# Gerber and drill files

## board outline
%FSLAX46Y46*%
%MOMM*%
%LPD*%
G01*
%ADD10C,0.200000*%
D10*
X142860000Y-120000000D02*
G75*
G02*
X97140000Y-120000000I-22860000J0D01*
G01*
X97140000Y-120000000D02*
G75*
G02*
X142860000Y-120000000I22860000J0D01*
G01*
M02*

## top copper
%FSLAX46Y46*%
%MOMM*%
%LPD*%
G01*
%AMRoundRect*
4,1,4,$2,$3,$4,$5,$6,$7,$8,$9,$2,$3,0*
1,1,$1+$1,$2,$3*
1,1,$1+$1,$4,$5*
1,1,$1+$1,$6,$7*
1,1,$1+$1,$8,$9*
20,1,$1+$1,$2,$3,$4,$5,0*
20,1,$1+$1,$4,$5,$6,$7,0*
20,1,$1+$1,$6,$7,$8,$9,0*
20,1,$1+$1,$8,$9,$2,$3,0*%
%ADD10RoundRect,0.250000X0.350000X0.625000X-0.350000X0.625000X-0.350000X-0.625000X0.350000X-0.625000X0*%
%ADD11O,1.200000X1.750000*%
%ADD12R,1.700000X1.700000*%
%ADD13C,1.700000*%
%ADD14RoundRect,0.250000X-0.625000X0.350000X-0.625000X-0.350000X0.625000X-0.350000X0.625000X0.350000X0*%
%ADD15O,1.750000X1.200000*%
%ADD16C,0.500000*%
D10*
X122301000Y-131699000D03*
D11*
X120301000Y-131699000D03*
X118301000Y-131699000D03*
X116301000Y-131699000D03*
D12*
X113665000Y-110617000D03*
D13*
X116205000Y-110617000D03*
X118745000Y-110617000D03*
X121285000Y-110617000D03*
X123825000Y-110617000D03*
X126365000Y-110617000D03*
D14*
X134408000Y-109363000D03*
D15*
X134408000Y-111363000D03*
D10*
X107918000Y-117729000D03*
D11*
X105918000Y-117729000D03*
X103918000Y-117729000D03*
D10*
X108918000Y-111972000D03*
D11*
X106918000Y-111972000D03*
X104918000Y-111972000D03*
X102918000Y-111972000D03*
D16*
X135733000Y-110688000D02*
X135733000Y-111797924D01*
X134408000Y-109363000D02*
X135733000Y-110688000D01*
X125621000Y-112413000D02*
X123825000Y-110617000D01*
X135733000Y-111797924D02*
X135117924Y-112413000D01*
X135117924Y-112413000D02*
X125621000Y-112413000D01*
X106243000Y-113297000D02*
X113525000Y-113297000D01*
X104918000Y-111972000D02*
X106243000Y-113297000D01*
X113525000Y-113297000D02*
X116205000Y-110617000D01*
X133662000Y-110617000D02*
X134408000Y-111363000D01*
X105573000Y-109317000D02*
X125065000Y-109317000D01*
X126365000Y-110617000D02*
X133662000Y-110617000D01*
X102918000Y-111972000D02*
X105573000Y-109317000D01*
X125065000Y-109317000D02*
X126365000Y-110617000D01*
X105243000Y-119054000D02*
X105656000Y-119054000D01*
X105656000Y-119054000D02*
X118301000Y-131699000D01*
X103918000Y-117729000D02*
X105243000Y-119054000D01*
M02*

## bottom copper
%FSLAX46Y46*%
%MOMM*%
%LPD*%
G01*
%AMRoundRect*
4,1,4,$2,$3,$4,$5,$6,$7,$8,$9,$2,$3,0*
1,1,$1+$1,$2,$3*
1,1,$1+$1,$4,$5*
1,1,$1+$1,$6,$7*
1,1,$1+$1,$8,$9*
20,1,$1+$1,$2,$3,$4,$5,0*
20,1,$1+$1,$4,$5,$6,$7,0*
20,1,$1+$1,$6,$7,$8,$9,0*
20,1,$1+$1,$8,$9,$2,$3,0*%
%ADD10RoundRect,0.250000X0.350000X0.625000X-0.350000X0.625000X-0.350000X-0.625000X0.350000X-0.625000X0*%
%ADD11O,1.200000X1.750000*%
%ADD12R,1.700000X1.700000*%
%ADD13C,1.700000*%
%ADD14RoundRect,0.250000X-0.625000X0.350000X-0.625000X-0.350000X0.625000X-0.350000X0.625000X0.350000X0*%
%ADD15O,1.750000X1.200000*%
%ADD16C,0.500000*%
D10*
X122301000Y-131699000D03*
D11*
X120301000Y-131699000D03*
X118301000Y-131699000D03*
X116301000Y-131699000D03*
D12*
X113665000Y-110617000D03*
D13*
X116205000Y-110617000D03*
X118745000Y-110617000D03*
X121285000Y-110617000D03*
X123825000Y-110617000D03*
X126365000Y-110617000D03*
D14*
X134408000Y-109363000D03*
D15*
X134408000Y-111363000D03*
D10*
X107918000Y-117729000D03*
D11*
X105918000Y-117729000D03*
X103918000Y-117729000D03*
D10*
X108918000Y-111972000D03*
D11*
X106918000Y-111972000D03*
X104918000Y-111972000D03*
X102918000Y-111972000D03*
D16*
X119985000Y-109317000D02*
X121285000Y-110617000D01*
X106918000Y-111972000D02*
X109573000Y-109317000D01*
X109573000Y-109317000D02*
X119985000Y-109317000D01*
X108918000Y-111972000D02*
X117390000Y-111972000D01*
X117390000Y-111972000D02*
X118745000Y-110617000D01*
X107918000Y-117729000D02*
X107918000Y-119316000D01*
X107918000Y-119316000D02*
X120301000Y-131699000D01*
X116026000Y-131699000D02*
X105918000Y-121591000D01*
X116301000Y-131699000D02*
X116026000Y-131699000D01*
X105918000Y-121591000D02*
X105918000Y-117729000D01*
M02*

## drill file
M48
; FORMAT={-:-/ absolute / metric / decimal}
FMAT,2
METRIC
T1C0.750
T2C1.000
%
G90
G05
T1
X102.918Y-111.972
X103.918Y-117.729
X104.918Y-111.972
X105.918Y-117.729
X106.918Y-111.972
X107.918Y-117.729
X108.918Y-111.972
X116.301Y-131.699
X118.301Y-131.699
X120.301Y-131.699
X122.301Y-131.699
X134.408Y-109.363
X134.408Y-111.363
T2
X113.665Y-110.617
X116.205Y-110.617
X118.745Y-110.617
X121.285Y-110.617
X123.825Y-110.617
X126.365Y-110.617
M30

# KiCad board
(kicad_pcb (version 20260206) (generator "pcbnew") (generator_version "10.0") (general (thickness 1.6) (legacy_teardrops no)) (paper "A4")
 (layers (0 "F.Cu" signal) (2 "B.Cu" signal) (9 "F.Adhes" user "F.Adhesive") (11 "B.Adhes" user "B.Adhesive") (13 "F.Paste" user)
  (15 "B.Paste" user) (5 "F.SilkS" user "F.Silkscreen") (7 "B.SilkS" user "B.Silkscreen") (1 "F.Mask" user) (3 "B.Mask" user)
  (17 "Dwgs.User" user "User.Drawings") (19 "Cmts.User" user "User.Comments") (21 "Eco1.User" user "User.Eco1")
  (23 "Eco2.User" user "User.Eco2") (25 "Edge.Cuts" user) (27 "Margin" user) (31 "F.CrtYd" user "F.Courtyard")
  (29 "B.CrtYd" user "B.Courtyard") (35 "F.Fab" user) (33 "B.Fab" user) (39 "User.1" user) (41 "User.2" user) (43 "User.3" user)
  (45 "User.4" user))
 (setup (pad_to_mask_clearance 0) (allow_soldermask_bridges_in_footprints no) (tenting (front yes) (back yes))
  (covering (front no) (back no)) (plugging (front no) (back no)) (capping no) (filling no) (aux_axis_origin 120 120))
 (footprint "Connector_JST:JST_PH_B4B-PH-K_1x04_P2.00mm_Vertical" (layer "F.Cu") (at 122.301 131.699 180)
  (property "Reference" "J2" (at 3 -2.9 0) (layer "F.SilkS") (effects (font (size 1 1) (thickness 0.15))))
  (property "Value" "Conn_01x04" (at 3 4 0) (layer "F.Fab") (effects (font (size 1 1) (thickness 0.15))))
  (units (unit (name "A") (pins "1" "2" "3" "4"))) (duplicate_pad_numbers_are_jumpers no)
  (pad "1" thru_hole roundrect (at 0 0 180) (size 1.2 1.75) (drill 0.75) (layers "*.Cu" "*.Mask") (remove_unused_layers no)
   (roundrect_rratio 0.208333) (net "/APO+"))
  (pad "2" thru_hole oval (at 2 0 180) (size 1.2 1.75) (drill 0.75) (layers "*.Cu" "*.Mask") (remove_unused_layers no) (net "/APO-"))
  (pad "3" thru_hole oval (at 4 0 180) (size 1.2 1.75) (drill 0.75) (layers "*.Cu" "*.Mask") (remove_unused_layers no) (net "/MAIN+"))
  (pad "4" thru_hole oval (at 6 0 180) (size 1.2 1.75) (drill 0.75) (layers "*.Cu" "*.Mask") (remove_unused_layers no) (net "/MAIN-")))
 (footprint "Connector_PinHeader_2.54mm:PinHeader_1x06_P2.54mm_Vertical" (layer "F.Cu") (at 113.665 110.617 90)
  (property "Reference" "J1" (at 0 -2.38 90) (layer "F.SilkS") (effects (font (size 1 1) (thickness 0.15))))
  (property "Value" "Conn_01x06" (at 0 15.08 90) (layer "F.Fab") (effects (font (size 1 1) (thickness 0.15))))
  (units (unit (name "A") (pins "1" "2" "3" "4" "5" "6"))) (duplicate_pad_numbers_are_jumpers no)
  (pad "1" thru_hole rect (at 0 0 90) (size 1.7 1.7) (drill 1) (layers "*.Cu" "*.Mask") (remove_unused_layers no) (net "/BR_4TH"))
  (pad "2" thru_hole circle (at 0 2.54 90) (size 1.7 1.7) (drill 1) (layers "*.Cu" "*.Mask") (remove_unused_layers no) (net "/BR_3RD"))
  (pad "3" thru_hole circle (at 0 5.08 90) (size 1.7 1.7) (drill 1) (layers "*.Cu" "*.Mask") (remove_unused_layers no) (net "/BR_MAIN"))
  (pad "4" thru_hole circle (at 0 7.62 90) (size 1.7 1.7) (drill 1) (layers "*.Cu" "*.Mask") (remove_unused_layers no) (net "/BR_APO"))
  (pad "5" thru_hole circle (at 0 10.16 90) (size 1.7 1.7) (drill 1) (layers "*.Cu" "*.Mask") (remove_unused_layers no) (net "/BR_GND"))
  (pad "6" thru_hole circle (at 0 12.7 90) (size 1.7 1.7) (drill 1) (layers "*.Cu" "*.Mask") (remove_unused_layers no) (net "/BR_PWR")))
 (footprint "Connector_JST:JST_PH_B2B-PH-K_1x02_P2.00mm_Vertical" (layer "F.Cu") (at 134.408 109.363 -90)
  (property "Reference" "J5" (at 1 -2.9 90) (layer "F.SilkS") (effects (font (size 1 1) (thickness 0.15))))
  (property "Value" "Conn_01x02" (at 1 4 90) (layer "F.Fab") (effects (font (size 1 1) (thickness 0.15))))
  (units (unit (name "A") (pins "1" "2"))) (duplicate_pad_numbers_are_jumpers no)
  (pad "1" thru_hole roundrect (at 0 0 270) (size 1.2 1.75) (drill 0.75) (layers "*.Cu" "*.Mask") (remove_unused_layers no)
   (roundrect_rratio 0.208333) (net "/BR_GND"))
  (pad "2" thru_hole oval (at 2 0 270) (size 1.2 1.75) (drill 0.75) (layers "*.Cu" "*.Mask") (remove_unused_layers no) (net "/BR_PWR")))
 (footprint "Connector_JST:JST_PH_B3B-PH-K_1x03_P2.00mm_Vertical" (layer "B.Cu") (at 107.918 117.729 180)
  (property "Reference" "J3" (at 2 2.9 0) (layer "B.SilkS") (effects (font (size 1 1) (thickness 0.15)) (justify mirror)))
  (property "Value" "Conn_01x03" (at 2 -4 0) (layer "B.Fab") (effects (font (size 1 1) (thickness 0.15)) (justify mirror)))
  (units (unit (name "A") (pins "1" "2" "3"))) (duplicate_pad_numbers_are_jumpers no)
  (pad "1" thru_hole roundrect (at 0 0 180) (size 1.2 1.75) (drill 0.75) (layers "*.Cu" "*.Mask") (remove_unused_layers no)
   (roundrect_rratio 0.208333) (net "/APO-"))
  (pad "2" thru_hole oval (at 2 0 180) (size 1.2 1.75) (drill 0.75) (layers "*.Cu" "*.Mask") (remove_unused_layers no) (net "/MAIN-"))
  (pad "3" thru_hole oval (at 4 0 180) (size 1.2 1.75) (drill 0.75) (layers "*.Cu" "*.Mask") (remove_unused_layers no) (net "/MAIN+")))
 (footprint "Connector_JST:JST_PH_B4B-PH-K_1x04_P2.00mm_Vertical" (layer "B.Cu") (at 108.918 111.972 180)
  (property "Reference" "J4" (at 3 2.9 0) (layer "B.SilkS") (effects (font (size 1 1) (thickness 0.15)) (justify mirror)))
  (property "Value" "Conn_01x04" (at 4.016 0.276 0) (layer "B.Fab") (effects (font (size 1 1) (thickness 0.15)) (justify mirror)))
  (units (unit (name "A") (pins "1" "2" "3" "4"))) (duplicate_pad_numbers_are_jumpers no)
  (pad "1" thru_hole roundrect (at 0 0 180) (size 1.2 1.75) (drill 0.75) (layers "*.Cu" "*.Mask") (remove_unused_layers no)
   (roundrect_rratio 0.208333) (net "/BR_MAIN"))
  (pad "2" thru_hole oval (at 2 0 180) (size 1.2 1.75) (drill 0.75) (layers "*.Cu" "*.Mask") (remove_unused_layers no) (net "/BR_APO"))
  (pad "3" thru_hole oval (at 4 0 180) (size 1.2 1.75) (drill 0.75) (layers "*.Cu" "*.Mask") (remove_unused_layers no) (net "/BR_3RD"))
  (pad "4" thru_hole oval (at 6 0 180) (size 1.2 1.75) (drill 0.75) (layers "*.Cu" "*.Mask") (remove_unused_layers no) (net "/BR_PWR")))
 (gr_circle (center 120 120) (end 120 142.86) (stroke (width 0.2) (type solid)) (fill no) (layer "Edge.Cuts"))
 (segment (start 135.733 110.688) (end 135.733 111.797924) (width 0.5) (layer "F.Cu") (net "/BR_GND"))
 (segment (start 134.408 109.363) (end 135.733 110.688) (width 0.5) (layer "F.Cu") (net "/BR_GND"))
 (segment (start 125.621 112.413) (end 123.825 110.617) (width 0.5) (layer "F.Cu") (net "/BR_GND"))
 (segment (start 135.733 111.797924) (end 135.117924 112.413) (width 0.5) (layer "F.Cu") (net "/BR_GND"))
 (segment (start 135.117924 112.413) (end 125.621 112.413) (width 0.5) (layer "F.Cu") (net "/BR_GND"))
 (segment (start 106.243 113.297) (end 113.525 113.297) (width 0.5) (layer "F.Cu") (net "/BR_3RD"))
 (segment (start 104.918 111.972) (end 106.243 113.297) (width 0.5) (layer "F.Cu") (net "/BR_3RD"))
 (segment (start 113.525 113.297) (end 116.205 110.617) (width 0.5) (layer "F.Cu") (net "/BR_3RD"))
 (segment (start 119.985 109.317) (end 121.285 110.617) (width 0.5) (layer "B.Cu") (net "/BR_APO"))
 (segment (start 106.918 111.972) (end 109.573 109.317) (width 0.5) (layer "B.Cu") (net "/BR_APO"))
 (segment (start 109.573 109.317) (end 119.985 109.317) (width 0.5) (layer "B.Cu") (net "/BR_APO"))
 (segment (start 108.918 111.972) (end 117.39 111.972) (width 0.5) (layer "B.Cu") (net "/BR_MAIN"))
 (segment (start 117.39 111.972) (end 118.745 110.617) (width 0.5) (layer "B.Cu") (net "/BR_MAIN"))
 (segment (start 133.662 110.617) (end 134.408 111.363) (width 0.5) (layer "F.Cu") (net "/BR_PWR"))
 (segment (start 105.573 109.317) (end 125.065 109.317) (width 0.5) (layer "F.Cu") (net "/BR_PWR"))
 (segment (start 126.365 110.617) (end 133.662 110.617) (width 0.5) (layer "F.Cu") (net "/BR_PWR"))
 (segment (start 102.918 111.972) (end 105.573 109.317) (width 0.5) (layer "F.Cu") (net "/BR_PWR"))
 (segment (start 125.065 109.317) (end 126.365 110.617) (width 0.5) (layer "F.Cu") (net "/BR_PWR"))
 (segment (start 107.918 117.729) (end 107.918 119.316) (width 0.5) (layer "B.Cu") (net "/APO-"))
 (segment (start 107.918 119.316) (end 120.301 131.699) (width 0.5) (layer "B.Cu") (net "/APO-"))
 (segment (start 116.026 131.699) (end 105.918 121.591) (width 0.5) (layer "B.Cu") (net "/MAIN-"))
 (segment (start 116.301 131.699) (end 116.026 131.699) (width 0.5) (layer "B.Cu") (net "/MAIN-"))
 (segment (start 105.918 121.591) (end 105.918 117.729) (width 0.5) (layer "B.Cu") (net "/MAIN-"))
 (segment (start 105.243 119.054) (end 105.656 119.054) (width 0.5) (layer "F.Cu") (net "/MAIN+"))
 (segment (start 105.656 119.054) (end 118.301 131.699) (width 0.5) (layer "F.Cu") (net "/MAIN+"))
 (segment (start 103.918 117.729) (end 105.243 119.054) (width 0.5) (layer "F.Cu") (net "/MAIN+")))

